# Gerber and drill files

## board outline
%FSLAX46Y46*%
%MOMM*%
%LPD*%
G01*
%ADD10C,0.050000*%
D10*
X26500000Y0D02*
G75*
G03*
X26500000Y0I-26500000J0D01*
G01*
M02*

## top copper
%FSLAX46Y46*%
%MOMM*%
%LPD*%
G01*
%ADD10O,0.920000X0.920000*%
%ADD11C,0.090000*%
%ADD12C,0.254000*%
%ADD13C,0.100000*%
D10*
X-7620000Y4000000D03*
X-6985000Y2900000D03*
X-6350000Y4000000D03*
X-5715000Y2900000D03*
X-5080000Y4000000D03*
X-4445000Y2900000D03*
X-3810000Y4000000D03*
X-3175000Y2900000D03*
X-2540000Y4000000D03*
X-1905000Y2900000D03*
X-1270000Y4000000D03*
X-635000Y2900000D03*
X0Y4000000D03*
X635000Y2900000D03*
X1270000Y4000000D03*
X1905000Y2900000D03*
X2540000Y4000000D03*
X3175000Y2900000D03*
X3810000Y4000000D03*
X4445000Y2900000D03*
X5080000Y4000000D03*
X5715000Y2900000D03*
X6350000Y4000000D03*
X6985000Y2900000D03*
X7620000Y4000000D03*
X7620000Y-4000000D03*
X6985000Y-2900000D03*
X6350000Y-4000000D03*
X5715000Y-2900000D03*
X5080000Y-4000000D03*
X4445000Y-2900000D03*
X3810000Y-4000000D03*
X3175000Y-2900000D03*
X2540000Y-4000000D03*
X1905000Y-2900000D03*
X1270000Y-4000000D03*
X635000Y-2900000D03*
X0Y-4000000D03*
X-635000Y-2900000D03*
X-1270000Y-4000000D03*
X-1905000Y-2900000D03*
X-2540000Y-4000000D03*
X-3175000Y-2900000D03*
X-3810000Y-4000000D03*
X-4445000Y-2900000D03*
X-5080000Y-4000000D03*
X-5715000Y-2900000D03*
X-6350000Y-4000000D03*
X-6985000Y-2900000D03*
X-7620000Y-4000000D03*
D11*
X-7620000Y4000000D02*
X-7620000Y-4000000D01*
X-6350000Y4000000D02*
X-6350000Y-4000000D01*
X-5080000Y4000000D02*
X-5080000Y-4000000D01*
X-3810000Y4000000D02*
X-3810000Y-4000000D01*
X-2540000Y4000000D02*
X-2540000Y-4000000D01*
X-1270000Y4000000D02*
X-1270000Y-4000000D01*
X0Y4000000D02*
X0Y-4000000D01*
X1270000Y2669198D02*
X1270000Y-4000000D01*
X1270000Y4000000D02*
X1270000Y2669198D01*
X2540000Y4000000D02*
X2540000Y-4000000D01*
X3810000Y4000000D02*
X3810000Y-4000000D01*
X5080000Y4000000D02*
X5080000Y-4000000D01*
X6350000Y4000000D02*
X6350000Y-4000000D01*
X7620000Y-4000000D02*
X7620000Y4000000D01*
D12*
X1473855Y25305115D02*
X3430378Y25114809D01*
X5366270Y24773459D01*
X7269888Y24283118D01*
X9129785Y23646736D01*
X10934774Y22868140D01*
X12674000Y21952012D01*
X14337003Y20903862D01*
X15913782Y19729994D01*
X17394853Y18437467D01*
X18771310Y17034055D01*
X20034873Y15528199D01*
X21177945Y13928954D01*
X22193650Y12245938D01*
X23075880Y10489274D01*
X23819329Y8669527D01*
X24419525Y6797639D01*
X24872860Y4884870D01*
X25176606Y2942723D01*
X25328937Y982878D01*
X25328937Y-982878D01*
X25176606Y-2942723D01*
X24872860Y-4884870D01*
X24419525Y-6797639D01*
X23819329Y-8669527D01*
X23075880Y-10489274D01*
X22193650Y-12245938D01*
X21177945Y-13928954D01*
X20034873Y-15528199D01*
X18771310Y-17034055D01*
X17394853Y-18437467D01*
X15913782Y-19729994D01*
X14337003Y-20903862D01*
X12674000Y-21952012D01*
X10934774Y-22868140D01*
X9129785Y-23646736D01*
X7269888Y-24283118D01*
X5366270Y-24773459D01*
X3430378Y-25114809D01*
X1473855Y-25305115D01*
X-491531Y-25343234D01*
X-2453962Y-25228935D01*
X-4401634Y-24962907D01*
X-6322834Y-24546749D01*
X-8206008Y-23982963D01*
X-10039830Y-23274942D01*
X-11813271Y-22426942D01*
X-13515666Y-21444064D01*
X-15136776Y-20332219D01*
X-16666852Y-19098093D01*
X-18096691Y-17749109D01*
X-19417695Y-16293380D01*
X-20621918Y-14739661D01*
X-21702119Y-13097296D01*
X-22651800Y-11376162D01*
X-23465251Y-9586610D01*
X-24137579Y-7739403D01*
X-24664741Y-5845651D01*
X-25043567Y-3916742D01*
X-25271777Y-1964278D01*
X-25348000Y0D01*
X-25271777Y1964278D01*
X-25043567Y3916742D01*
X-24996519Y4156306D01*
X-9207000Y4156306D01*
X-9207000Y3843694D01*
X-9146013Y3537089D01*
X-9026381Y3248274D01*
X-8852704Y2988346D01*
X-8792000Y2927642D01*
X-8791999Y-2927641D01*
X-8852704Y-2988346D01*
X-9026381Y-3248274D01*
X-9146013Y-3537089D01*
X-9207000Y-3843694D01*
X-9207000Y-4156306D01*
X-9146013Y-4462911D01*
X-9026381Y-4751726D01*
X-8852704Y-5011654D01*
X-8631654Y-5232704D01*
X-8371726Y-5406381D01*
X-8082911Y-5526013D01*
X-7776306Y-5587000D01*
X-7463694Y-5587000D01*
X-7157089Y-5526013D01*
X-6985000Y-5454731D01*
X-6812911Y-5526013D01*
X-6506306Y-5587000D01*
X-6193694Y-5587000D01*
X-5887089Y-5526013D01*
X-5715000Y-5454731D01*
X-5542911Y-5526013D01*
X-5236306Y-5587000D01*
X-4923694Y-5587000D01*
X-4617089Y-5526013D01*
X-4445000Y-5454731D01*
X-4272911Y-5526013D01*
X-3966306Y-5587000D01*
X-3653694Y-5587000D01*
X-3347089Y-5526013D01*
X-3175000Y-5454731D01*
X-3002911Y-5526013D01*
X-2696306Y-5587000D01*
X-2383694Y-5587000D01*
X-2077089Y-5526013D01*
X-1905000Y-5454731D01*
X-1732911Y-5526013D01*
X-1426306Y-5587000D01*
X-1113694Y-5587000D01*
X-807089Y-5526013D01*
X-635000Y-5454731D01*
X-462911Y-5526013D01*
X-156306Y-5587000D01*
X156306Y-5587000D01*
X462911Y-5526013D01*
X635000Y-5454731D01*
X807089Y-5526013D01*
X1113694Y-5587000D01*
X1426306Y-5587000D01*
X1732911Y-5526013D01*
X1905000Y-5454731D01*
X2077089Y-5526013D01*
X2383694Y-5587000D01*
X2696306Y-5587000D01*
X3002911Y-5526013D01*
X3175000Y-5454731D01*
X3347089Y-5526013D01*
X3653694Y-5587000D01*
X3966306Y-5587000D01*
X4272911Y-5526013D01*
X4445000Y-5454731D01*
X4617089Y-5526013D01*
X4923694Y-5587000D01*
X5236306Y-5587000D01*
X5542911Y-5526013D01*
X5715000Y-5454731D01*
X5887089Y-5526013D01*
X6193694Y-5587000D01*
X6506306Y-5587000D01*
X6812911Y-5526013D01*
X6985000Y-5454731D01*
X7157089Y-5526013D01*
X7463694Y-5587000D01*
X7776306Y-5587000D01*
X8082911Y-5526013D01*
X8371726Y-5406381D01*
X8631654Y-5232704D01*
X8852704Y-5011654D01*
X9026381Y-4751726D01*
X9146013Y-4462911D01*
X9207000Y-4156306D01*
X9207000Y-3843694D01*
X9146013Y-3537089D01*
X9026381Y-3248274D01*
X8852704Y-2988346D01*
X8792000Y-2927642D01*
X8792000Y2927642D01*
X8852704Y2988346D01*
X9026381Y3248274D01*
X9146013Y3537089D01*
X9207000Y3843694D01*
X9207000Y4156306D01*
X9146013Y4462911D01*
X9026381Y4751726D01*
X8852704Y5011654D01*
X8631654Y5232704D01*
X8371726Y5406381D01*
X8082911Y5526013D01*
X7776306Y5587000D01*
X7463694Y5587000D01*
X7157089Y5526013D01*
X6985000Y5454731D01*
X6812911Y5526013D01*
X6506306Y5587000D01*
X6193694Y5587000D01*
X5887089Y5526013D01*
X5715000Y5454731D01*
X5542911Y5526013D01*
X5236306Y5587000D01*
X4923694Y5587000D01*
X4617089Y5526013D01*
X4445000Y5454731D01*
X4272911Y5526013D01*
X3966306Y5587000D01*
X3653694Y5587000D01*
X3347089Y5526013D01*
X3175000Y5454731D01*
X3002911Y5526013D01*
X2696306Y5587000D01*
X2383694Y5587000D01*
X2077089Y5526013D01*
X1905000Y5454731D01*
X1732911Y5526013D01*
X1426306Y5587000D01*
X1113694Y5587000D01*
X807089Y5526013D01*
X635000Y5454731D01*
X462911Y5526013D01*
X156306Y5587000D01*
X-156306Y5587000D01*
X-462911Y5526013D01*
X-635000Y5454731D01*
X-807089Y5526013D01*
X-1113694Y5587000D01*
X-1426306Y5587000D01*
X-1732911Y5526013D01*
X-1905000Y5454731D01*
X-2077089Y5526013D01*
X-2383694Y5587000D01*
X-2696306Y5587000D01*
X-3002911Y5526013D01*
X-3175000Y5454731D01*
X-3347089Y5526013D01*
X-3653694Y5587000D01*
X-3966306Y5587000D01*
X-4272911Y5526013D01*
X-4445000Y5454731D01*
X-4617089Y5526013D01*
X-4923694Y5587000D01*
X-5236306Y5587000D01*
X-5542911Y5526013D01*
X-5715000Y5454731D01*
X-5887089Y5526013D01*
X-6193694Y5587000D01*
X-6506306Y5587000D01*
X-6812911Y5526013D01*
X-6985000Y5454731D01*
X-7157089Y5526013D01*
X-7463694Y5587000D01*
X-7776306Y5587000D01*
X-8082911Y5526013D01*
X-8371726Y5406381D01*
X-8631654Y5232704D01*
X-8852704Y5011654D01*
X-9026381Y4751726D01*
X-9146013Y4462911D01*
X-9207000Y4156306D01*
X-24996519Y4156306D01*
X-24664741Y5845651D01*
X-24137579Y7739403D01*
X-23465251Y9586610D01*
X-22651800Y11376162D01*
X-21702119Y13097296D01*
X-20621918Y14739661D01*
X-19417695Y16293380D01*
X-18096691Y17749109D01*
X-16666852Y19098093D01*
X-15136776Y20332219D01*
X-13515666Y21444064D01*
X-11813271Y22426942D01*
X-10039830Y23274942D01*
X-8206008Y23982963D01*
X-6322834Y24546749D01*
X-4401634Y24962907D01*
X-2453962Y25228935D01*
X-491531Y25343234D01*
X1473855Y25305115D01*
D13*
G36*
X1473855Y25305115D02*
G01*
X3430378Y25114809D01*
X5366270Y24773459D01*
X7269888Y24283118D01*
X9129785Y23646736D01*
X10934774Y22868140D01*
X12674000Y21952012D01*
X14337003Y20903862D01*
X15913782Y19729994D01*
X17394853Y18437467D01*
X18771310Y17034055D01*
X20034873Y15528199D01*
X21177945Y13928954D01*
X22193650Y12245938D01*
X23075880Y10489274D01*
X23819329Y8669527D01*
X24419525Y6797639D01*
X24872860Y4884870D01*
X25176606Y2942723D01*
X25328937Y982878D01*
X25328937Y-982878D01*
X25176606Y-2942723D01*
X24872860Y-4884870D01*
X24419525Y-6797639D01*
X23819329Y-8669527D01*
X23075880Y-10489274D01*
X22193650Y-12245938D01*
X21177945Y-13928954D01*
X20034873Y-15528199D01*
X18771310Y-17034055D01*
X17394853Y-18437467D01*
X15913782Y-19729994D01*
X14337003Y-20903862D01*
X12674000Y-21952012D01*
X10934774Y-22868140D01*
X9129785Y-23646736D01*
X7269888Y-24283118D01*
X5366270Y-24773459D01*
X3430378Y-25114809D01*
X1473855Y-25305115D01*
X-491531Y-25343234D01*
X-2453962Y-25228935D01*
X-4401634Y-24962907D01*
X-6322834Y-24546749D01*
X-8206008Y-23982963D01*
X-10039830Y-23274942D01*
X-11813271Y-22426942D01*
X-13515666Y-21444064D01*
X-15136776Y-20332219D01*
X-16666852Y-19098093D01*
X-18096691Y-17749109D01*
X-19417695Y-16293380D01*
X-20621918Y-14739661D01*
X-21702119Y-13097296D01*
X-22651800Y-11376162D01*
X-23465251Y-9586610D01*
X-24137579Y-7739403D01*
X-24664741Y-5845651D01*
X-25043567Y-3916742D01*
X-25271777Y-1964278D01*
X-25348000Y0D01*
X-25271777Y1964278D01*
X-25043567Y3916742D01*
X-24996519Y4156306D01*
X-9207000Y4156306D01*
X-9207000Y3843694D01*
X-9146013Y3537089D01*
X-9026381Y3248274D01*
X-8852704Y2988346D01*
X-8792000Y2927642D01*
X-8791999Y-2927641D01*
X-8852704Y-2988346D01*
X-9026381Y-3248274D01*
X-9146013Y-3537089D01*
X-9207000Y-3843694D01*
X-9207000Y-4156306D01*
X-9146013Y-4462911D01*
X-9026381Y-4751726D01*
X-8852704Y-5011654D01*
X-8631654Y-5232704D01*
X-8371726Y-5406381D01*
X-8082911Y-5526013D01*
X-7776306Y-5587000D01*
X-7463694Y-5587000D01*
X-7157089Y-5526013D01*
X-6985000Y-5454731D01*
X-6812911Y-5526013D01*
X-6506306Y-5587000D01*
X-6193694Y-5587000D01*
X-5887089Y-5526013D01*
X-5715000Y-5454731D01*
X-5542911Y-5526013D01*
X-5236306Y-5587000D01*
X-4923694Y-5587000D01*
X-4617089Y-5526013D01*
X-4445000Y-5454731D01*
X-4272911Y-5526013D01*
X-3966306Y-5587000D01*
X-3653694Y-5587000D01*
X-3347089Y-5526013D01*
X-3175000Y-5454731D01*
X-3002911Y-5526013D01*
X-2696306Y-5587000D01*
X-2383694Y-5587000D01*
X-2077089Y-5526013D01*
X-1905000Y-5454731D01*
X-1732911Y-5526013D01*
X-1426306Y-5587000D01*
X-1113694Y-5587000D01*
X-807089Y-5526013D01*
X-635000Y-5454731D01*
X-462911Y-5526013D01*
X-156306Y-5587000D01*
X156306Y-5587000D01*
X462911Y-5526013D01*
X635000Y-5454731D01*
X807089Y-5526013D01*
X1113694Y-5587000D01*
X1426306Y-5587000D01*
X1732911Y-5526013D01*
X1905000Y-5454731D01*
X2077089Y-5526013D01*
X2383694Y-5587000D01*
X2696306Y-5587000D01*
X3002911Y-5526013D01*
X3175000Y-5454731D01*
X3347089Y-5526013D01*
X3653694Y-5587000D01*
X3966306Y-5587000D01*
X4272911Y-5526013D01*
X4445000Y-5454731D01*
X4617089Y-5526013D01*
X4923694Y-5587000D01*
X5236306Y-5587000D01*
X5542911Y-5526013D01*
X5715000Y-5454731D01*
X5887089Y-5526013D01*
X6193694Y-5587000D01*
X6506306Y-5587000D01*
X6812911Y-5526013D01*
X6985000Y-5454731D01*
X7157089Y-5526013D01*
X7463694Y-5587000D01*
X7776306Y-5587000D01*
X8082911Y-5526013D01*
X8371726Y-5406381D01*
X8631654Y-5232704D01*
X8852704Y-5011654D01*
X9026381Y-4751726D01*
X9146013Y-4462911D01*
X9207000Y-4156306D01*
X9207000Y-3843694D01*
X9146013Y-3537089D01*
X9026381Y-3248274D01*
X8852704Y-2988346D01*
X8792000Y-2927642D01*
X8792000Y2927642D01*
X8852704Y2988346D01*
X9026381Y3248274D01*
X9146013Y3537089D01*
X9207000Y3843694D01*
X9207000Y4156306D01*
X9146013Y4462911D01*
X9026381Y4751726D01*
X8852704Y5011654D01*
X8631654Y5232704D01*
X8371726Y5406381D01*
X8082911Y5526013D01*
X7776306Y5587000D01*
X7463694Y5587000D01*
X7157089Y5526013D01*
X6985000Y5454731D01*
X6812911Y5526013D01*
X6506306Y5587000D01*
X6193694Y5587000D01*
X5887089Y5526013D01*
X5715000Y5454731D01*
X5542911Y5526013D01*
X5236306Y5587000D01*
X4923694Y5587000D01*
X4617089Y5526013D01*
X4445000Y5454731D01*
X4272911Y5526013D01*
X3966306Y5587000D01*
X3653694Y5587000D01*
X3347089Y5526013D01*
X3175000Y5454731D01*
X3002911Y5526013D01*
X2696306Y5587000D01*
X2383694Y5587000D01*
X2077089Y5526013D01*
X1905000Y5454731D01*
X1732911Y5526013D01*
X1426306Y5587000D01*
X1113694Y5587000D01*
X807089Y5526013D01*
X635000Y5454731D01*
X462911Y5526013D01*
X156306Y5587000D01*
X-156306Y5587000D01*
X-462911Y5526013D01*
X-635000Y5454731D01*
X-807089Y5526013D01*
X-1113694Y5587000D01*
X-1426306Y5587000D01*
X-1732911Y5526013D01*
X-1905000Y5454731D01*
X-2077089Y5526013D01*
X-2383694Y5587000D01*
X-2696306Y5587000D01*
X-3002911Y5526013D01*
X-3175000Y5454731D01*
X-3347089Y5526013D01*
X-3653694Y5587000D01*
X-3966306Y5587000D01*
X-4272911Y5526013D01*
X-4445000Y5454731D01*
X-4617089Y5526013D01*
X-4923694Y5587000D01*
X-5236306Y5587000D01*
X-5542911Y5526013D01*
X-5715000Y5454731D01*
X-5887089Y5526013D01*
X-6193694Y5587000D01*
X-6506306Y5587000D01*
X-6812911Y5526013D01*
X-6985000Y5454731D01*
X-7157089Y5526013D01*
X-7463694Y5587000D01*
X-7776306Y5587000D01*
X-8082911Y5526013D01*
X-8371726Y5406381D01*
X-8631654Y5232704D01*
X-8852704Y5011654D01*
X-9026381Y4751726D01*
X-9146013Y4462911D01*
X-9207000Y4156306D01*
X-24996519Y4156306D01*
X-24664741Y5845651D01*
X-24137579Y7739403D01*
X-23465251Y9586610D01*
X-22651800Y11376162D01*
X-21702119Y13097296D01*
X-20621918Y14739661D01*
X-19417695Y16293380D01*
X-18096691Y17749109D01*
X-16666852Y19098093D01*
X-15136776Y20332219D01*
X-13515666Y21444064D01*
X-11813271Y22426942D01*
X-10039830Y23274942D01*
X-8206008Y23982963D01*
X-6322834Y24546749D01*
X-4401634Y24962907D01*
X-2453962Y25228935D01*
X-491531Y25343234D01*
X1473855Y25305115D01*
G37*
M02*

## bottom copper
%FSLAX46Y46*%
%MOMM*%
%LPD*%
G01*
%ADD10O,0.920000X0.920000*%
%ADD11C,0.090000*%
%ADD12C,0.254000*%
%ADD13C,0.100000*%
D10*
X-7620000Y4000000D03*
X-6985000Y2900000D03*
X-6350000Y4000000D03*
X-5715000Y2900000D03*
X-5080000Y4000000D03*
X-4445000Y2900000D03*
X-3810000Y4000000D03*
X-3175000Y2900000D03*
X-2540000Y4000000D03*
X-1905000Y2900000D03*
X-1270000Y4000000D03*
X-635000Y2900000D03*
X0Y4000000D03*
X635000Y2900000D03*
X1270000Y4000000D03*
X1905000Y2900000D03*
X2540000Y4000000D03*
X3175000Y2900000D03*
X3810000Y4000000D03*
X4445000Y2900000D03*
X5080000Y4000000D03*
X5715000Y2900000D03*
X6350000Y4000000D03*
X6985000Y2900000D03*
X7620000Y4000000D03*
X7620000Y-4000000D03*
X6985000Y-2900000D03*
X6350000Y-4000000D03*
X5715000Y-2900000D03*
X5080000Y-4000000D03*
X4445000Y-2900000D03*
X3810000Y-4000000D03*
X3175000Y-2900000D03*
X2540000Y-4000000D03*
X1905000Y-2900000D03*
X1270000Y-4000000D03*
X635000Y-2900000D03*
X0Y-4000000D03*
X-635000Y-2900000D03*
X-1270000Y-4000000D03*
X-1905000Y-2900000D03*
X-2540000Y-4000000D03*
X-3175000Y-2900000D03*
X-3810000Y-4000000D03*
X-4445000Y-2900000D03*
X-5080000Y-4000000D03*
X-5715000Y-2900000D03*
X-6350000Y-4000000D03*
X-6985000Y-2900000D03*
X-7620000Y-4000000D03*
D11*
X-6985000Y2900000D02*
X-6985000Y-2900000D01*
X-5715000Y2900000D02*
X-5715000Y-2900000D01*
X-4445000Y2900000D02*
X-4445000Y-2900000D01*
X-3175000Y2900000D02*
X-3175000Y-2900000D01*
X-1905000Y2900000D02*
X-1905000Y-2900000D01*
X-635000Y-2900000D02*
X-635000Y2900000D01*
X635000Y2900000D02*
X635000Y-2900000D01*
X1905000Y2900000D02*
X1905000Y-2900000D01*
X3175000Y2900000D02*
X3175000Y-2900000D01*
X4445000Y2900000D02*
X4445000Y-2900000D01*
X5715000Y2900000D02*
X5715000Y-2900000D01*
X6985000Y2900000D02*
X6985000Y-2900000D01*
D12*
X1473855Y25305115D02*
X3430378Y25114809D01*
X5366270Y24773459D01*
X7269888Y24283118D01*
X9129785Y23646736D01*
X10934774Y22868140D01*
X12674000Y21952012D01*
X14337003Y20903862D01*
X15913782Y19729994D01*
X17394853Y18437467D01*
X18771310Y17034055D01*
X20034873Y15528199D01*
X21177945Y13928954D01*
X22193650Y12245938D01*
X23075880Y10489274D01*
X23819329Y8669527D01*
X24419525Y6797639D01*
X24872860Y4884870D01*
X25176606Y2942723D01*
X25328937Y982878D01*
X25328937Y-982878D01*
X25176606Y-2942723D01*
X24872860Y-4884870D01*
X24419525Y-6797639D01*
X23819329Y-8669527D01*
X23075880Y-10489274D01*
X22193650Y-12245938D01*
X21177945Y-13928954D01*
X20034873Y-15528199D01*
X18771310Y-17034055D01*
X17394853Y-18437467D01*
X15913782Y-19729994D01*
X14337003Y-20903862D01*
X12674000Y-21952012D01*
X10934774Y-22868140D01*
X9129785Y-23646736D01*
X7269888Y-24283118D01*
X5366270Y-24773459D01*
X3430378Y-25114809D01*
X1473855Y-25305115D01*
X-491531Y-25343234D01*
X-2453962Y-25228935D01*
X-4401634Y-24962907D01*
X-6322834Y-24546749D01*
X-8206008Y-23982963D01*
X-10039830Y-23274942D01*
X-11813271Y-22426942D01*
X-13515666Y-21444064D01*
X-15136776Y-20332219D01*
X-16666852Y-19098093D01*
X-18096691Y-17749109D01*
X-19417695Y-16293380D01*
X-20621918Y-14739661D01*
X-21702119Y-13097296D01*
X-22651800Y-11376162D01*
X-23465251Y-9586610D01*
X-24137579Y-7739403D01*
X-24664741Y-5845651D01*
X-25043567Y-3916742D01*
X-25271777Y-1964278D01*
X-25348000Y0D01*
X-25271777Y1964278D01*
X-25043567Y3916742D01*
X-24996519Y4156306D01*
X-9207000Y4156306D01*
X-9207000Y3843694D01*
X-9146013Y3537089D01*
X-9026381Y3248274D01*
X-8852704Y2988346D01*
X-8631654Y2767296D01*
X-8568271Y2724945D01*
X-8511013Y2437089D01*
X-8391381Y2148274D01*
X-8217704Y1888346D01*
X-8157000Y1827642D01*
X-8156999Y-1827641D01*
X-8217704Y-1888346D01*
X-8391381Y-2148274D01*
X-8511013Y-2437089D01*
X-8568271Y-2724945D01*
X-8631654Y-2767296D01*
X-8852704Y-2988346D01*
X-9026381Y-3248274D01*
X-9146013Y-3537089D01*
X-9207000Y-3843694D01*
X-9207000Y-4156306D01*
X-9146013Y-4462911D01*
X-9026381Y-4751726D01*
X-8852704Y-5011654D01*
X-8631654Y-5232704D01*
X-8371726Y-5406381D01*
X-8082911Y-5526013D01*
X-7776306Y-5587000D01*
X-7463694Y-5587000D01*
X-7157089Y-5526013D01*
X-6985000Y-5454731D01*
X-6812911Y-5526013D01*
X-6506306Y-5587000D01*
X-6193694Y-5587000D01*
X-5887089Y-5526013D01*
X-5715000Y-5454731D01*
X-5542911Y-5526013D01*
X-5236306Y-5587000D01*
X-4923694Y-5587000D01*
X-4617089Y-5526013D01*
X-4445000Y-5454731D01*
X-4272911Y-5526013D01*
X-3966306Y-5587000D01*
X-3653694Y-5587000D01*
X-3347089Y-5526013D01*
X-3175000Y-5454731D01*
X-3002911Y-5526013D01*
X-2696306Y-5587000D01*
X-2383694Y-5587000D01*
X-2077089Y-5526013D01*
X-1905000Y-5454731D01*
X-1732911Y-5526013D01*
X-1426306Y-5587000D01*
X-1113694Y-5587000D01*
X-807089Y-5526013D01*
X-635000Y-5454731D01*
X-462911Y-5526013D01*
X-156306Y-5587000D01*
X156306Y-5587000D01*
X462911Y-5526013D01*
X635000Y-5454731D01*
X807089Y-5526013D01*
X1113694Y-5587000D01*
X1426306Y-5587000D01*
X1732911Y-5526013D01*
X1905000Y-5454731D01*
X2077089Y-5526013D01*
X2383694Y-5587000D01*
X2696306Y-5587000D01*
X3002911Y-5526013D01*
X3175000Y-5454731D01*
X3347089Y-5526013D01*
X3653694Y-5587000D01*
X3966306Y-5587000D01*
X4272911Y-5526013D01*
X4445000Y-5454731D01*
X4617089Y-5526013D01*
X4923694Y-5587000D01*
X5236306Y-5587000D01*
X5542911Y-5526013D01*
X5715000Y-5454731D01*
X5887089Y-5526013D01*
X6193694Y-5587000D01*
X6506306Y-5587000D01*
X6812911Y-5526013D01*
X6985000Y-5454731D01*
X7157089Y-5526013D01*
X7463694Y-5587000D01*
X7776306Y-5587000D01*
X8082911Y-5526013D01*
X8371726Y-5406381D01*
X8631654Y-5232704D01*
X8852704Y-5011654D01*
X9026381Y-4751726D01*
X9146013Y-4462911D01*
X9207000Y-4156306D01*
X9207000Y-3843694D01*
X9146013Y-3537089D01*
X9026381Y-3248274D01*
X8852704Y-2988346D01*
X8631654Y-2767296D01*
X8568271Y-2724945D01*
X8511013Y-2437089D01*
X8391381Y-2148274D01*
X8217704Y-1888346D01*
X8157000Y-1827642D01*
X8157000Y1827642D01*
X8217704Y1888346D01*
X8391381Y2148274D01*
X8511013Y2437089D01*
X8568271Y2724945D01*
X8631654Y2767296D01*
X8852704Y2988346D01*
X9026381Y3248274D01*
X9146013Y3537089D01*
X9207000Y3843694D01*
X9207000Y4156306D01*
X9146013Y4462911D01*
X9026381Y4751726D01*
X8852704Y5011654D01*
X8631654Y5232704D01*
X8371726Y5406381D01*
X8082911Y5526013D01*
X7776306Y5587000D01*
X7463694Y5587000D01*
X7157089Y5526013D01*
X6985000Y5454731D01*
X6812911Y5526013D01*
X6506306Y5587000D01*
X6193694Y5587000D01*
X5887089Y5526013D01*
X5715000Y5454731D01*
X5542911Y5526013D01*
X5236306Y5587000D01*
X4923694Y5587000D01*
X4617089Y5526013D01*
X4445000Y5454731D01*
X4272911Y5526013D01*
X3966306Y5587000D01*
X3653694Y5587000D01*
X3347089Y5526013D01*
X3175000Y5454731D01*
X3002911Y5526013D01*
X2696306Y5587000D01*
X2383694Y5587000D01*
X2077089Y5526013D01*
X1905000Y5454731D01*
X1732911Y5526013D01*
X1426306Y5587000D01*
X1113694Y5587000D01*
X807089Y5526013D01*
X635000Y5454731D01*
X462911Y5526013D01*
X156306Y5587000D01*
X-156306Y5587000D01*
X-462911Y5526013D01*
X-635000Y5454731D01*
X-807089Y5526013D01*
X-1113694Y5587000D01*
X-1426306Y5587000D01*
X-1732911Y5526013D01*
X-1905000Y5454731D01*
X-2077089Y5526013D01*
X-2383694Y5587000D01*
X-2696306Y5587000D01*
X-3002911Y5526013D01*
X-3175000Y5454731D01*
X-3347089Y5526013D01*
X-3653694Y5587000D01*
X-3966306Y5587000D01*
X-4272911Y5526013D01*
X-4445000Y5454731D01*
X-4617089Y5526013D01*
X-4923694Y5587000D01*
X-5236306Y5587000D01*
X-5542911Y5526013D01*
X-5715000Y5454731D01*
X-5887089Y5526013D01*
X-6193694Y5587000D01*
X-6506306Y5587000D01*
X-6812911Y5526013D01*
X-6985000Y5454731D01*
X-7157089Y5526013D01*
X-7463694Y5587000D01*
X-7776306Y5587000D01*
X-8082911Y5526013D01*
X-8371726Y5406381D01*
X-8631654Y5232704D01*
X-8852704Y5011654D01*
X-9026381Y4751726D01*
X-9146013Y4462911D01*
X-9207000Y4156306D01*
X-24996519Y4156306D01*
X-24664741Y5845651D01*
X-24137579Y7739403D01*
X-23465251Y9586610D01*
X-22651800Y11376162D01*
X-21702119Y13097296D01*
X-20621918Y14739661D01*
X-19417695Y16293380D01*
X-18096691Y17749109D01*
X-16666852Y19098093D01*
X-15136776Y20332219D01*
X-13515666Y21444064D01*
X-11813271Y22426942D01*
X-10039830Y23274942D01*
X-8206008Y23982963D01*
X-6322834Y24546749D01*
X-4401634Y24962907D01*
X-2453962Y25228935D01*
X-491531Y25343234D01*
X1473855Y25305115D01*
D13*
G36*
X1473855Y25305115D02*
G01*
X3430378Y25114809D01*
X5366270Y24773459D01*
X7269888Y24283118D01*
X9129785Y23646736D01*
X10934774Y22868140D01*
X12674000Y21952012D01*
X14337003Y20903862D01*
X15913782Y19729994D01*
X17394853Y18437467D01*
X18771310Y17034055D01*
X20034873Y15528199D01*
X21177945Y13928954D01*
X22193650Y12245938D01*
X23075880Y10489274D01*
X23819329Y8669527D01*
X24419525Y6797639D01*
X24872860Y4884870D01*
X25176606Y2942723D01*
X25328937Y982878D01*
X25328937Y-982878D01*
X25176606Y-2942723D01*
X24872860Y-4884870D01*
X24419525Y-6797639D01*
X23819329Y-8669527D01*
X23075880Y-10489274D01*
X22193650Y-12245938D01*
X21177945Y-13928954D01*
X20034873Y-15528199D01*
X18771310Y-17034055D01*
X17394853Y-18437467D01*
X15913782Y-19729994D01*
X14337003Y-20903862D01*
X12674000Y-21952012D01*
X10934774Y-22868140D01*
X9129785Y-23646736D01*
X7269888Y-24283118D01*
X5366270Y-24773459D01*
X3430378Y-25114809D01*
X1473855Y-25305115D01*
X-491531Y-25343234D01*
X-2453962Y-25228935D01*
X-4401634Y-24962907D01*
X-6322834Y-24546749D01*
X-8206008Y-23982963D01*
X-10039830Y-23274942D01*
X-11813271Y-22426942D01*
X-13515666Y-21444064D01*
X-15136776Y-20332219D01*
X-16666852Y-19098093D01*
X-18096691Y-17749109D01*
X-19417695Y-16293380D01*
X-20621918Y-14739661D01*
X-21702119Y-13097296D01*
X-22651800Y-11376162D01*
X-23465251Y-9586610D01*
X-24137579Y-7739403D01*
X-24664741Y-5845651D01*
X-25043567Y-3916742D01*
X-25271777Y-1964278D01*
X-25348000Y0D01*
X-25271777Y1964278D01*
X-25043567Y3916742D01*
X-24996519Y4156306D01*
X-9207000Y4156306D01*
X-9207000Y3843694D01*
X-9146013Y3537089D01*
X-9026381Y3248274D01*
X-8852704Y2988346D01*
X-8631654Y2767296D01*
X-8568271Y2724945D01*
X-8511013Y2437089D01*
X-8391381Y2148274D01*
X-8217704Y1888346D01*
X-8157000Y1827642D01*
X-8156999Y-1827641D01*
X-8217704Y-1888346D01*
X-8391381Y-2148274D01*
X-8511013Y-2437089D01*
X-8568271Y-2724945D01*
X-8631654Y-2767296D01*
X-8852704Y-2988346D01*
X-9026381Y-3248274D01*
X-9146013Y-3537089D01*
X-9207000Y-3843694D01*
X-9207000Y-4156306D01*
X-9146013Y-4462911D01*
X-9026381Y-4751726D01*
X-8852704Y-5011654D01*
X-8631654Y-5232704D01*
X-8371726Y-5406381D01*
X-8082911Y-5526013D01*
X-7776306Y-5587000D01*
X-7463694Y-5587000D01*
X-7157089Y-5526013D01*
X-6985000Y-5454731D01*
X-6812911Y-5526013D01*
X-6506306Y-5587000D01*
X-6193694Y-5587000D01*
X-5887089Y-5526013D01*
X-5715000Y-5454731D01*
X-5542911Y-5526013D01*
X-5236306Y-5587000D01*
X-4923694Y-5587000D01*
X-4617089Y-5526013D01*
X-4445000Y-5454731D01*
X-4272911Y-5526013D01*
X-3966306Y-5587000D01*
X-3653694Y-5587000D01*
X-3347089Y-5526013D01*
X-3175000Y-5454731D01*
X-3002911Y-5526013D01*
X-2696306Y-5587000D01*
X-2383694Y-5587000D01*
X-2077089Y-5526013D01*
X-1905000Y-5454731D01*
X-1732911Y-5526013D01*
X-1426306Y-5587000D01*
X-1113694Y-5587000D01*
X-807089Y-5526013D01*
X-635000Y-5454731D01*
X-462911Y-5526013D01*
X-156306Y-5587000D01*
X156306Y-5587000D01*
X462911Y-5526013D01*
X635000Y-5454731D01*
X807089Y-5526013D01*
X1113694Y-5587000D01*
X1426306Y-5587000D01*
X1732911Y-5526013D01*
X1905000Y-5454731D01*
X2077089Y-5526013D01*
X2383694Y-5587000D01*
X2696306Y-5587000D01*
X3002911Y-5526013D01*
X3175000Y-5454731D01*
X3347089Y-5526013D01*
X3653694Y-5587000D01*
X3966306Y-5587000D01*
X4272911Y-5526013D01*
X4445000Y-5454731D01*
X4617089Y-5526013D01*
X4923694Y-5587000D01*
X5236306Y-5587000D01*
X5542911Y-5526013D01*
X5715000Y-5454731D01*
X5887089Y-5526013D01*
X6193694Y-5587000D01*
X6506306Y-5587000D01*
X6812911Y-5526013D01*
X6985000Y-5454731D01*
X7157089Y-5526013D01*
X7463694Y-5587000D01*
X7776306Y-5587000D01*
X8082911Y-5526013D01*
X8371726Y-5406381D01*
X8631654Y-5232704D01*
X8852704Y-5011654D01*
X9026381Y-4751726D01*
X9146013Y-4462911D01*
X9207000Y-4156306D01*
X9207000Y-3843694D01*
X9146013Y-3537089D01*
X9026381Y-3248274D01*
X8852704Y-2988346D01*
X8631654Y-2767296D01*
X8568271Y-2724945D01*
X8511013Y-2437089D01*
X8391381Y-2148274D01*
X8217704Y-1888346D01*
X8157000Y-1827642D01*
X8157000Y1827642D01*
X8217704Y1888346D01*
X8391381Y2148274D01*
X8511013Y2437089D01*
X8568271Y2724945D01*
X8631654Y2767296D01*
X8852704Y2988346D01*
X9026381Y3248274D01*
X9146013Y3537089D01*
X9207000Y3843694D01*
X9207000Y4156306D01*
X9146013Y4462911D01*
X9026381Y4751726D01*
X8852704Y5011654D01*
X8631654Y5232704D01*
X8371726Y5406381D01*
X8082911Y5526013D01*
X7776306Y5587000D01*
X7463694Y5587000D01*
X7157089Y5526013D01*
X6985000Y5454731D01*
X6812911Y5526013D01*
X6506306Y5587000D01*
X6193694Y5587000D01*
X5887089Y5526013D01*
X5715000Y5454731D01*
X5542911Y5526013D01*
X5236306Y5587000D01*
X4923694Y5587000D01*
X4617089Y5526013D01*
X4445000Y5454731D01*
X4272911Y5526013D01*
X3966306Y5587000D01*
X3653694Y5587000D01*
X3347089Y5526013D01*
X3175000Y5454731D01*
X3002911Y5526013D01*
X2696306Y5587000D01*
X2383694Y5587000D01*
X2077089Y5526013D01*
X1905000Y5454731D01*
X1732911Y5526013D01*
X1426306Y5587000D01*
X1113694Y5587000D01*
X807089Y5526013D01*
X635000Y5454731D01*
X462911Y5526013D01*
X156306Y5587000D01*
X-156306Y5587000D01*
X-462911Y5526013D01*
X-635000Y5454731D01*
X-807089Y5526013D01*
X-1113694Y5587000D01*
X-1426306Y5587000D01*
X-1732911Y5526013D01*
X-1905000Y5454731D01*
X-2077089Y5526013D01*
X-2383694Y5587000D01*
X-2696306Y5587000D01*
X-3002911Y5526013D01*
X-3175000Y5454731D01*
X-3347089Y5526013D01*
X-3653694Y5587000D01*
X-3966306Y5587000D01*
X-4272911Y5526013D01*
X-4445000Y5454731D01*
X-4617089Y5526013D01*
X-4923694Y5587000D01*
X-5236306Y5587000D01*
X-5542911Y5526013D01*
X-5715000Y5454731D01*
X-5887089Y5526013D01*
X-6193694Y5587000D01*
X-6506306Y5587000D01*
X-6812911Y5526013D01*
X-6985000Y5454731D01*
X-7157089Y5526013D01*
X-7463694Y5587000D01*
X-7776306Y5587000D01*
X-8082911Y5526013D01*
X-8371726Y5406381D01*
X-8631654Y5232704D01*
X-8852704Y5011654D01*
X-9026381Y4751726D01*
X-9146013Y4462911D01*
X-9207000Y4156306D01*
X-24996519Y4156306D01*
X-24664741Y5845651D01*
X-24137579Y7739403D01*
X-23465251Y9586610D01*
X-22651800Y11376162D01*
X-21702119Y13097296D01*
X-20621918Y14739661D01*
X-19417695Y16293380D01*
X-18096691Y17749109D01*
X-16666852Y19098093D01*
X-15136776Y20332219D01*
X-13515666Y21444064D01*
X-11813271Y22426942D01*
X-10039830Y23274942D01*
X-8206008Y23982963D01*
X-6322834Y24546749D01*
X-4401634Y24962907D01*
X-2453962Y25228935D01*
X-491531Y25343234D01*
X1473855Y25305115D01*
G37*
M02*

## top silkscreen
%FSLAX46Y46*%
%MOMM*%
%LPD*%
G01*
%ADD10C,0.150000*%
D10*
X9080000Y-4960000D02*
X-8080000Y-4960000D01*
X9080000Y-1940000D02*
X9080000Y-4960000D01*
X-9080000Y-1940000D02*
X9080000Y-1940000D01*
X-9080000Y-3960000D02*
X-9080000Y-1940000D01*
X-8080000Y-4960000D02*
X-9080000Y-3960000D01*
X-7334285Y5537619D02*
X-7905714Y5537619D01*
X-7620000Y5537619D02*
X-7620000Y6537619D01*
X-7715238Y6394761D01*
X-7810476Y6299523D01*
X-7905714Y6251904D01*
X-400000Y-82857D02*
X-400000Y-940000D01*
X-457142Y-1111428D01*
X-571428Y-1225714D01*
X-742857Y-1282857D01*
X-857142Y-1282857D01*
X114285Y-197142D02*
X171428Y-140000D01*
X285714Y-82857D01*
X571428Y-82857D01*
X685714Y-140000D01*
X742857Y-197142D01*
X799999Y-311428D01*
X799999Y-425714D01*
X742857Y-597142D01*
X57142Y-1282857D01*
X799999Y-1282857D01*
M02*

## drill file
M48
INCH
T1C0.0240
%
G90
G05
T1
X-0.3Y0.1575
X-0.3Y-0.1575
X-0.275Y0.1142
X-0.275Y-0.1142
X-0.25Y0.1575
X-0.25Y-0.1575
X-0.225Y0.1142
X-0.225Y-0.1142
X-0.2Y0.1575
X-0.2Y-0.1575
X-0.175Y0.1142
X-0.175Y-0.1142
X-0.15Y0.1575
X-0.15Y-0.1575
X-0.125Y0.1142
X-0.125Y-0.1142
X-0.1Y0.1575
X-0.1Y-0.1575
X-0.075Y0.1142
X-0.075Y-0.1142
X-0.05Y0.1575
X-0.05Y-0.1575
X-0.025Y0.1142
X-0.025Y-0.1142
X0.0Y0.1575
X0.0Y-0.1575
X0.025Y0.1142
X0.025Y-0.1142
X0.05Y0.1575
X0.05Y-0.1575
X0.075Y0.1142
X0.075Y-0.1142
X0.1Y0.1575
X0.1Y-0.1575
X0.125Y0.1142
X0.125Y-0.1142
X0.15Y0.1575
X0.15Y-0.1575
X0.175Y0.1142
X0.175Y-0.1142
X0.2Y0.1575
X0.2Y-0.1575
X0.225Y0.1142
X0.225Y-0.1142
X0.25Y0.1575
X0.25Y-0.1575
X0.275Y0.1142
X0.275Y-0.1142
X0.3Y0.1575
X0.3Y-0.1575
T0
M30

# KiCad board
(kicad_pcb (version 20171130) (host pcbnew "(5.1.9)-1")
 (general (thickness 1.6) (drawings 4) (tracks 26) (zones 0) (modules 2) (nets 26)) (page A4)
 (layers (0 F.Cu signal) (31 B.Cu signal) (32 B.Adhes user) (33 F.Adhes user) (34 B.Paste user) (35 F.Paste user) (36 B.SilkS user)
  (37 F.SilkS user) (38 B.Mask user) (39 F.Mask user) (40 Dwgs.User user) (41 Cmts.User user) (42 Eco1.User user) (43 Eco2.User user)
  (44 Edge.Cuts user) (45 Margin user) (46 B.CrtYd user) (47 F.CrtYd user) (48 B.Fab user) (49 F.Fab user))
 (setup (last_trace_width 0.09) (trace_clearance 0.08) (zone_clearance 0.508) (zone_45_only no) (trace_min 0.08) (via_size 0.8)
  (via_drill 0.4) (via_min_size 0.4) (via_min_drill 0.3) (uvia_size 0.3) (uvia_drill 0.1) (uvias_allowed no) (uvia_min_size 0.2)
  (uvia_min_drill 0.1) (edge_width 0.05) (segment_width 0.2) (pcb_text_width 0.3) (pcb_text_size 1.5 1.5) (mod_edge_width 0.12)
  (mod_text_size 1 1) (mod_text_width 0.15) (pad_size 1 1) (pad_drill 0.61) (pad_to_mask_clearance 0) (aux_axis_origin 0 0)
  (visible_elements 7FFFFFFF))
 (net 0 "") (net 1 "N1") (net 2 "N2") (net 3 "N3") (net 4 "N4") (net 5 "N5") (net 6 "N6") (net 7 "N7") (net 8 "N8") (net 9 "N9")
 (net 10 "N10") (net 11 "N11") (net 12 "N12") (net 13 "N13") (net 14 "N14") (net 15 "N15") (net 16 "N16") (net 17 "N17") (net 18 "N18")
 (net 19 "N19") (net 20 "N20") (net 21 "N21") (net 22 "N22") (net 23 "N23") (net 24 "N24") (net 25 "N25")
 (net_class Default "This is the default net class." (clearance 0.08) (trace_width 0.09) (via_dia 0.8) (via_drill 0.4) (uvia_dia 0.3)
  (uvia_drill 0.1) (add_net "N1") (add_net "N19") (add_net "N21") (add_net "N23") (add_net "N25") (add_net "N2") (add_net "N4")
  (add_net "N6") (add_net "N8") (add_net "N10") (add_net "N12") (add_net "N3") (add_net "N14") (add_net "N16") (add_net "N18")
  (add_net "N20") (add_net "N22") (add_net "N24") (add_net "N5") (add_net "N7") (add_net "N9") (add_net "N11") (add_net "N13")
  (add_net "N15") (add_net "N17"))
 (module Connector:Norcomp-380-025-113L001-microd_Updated (layer F.Cu) (at 0 -3.45)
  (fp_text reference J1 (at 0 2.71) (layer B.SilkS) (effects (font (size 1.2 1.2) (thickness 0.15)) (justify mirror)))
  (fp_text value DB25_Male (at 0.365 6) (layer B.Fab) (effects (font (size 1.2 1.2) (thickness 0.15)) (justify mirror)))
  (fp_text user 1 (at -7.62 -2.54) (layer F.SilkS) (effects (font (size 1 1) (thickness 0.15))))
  (pad 1 thru_hole oval (at -7.62 -0.55) (size 0.92 0.92) (drill 0.61) (layers *.Cu *.Mask) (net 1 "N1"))
  (pad 14 thru_hole oval (at -6.985 0.55) (size 0.92 0.92) (drill 0.61) (layers *.Cu *.Mask) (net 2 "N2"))
  (pad 2 thru_hole oval (at -6.35 -0.55) (size 0.92 0.92) (drill 0.61) (layers *.Cu *.Mask) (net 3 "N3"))
  (pad 15 thru_hole oval (at -5.715 0.55) (size 0.92 0.92) (drill 0.61) (layers *.Cu *.Mask) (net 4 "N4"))
  (pad 3 thru_hole oval (at -5.08 -0.55) (size 0.92 0.92) (drill 0.61) (layers *.Cu *.Mask) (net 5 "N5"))
  (pad 16 thru_hole oval (at -4.445 0.55) (size 0.92 0.92) (drill 0.61) (layers *.Cu *.Mask) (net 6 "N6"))
  (pad 4 thru_hole oval (at -3.81 -0.55) (size 0.92 0.92) (drill 0.61) (layers *.Cu *.Mask) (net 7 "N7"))
  (pad 17 thru_hole oval (at -3.175 0.55) (size 0.92 0.92) (drill 0.61) (layers *.Cu *.Mask) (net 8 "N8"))
  (pad 5 thru_hole oval (at -2.54 -0.55) (size 0.92 0.92) (drill 0.61) (layers *.Cu *.Mask) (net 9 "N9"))
  (pad 18 thru_hole oval (at -1.905 0.55) (size 0.92 0.92) (drill 0.61) (layers *.Cu *.Mask) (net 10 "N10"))
  (pad 6 thru_hole oval (at -1.27 -0.55) (size 0.92 0.92) (drill 0.61) (layers *.Cu *.Mask) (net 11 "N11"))
  (pad 19 thru_hole oval (at -0.635 0.55) (size 0.92 0.92) (drill 0.61) (layers *.Cu *.Mask) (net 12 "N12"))
  (pad 7 thru_hole oval (at 0 -0.55) (size 0.92 0.92) (drill 0.61) (layers *.Cu *.Mask) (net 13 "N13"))
  (pad 20 thru_hole oval (at 0.635 0.55) (size 0.92 0.92) (drill 0.61) (layers *.Cu *.Mask) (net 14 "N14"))
  (pad 8 thru_hole oval (at 1.27 -0.55) (size 0.92 0.92) (drill 0.61) (layers *.Cu *.Mask) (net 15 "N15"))
  (pad 21 thru_hole oval (at 1.905 0.55) (size 0.92 0.92) (drill 0.61) (layers *.Cu *.Mask) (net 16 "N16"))
  (pad 9 thru_hole oval (at 2.54 -0.55) (size 0.92 0.92) (drill 0.61) (layers *.Cu *.Mask) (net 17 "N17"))
  (pad 22 thru_hole oval (at 3.175 0.55) (size 0.92 0.92) (drill 0.61) (layers *.Cu *.Mask) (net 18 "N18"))
  (pad 10 thru_hole oval (at 3.81 -0.55) (size 0.92 0.92) (drill 0.61) (layers *.Cu *.Mask) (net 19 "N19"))
  (pad 23 thru_hole oval (at 4.445 0.55) (size 0.92 0.92) (drill 0.61) (layers *.Cu *.Mask) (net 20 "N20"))
  (pad 11 thru_hole oval (at 5.08 -0.55) (size 0.92 0.92) (drill 0.61) (layers *.Cu *.Mask) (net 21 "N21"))
  (pad 24 thru_hole oval (at 5.715 0.55) (size 0.92 0.92) (drill 0.61) (layers *.Cu *.Mask) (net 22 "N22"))
  (pad 12 thru_hole oval (at 6.35 -0.55) (size 0.92 0.92) (drill 0.61) (layers *.Cu *.Mask) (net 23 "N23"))
  (pad 25 thru_hole oval (at 6.985 0.55) (size 0.92 0.92) (drill 0.61) (layers *.Cu *.Mask) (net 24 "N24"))
  (pad 13 thru_hole oval (at 7.62 -0.55) (size 0.92 0.92) (drill 0.61) (layers *.Cu *.Mask) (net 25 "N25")))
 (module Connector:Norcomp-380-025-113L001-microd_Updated (layer B.Cu) (at 0 3.45)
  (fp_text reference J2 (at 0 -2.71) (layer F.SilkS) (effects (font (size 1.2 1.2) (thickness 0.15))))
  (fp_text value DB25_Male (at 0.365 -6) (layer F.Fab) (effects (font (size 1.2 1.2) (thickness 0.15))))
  (fp_line (start 9.08 1.51) (end -8.08 1.51) (layer F.SilkS) (width 0.15))
  (fp_line (start 9.08 -1.51) (end 9.08 1.51) (layer F.SilkS) (width 0.15))
  (fp_line (start -9.08 -1.51) (end 9.08 -1.51) (layer F.SilkS) (width 0.15))
  (fp_line (start -9.08 0.51) (end -9.08 -1.51) (layer F.SilkS) (width 0.15))
  (fp_line (start -8.08 1.51) (end -9.08 0.51) (layer F.SilkS) (width 0.15))
  (pad 13 thru_hole oval (at 7.62 0.55) (size 0.92 0.92) (drill 0.61) (layers *.Cu *.Mask) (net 25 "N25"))
  (pad 25 thru_hole oval (at 6.985 -0.55) (size 0.92 0.92) (drill 0.61) (layers *.Cu *.Mask) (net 24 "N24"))
  (pad 12 thru_hole oval (at 6.35 0.55) (size 0.92 0.92) (drill 0.61) (layers *.Cu *.Mask) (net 23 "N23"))
  (pad 24 thru_hole oval (at 5.715 -0.55) (size 0.92 0.92) (drill 0.61) (layers *.Cu *.Mask) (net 22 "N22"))
  (pad 11 thru_hole oval (at 5.08 0.55) (size 0.92 0.92) (drill 0.61) (layers *.Cu *.Mask) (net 21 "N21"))
  (pad 23 thru_hole oval (at 4.445 -0.55) (size 0.92 0.92) (drill 0.61) (layers *.Cu *.Mask) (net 20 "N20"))
  (pad 10 thru_hole oval (at 3.81 0.55) (size 0.92 0.92) (drill 0.61) (layers *.Cu *.Mask) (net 19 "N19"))
  (pad 22 thru_hole oval (at 3.175 -0.55) (size 0.92 0.92) (drill 0.61) (layers *.Cu *.Mask) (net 18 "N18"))
  (pad 9 thru_hole oval (at 2.54 0.55) (size 0.92 0.92) (drill 0.61) (layers *.Cu *.Mask) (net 17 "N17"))
  (pad 21 thru_hole oval (at 1.905 -0.55) (size 0.92 0.92) (drill 0.61) (layers *.Cu *.Mask) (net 16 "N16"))
  (pad 8 thru_hole oval (at 1.27 0.55) (size 0.92 0.92) (drill 0.61) (layers *.Cu *.Mask) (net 15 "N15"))
  (pad 20 thru_hole oval (at 0.635 -0.55) (size 0.92 0.92) (drill 0.61) (layers *.Cu *.Mask) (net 14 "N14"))
  (pad 7 thru_hole oval (at 0 0.55) (size 0.92 0.92) (drill 0.61) (layers *.Cu *.Mask) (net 13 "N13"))
  (pad 19 thru_hole oval (at -0.635 -0.55) (size 0.92 0.92) (drill 0.61) (layers *.Cu *.Mask) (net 12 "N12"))
  (pad 6 thru_hole oval (at -1.27 0.55) (size 0.92 0.92) (drill 0.61) (layers *.Cu *.Mask) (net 11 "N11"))
  (pad 18 thru_hole oval (at -1.905 -0.55) (size 0.92 0.92) (drill 0.61) (layers *.Cu *.Mask) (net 10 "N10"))
  (pad 5 thru_hole oval (at -2.54 0.55) (size 0.92 0.92) (drill 0.61) (layers *.Cu *.Mask) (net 9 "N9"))
  (pad 17 thru_hole oval (at -3.175 -0.55) (size 0.92 0.92) (drill 0.61) (layers *.Cu *.Mask) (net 8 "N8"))
  (pad 4 thru_hole oval (at -3.81 0.55) (size 0.92 0.92) (drill 0.61) (layers *.Cu *.Mask) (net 7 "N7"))
  (pad 16 thru_hole oval (at -4.445 -0.55) (size 0.92 0.92) (drill 0.61) (layers *.Cu *.Mask) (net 6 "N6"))
  (pad 3 thru_hole oval (at -5.08 0.55) (size 0.92 0.92) (drill 0.61) (layers *.Cu *.Mask) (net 5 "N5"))
  (pad 15 thru_hole oval (at -5.715 -0.55) (size 0.92 0.92) (drill 0.61) (layers *.Cu *.Mask) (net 4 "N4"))
  (pad 2 thru_hole oval (at -6.35 0.55) (size 0.92 0.92) (drill 0.61) (layers *.Cu *.Mask) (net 3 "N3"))
  (pad 14 thru_hole oval (at -6.985 -0.55) (size 0.92 0.92) (drill 0.61) (layers *.Cu *.Mask) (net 2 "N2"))
  (pad 1 thru_hole oval (at -7.62 0.55) (size 0.92 0.92) (drill 0.61) (layers *.Cu *.Mask) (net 1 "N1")))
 (gr_circle (center 0 0) (end 26.5 0) (layer Edge.Cuts) (width 0.05))
 (segment (start -7.62 -4) (end -7.62 4) (width 0.09) (layer F.Cu) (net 1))
 (segment (start -6.985 -2.9) (end -6.985 2.9) (width 0.09) (layer B.Cu) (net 2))
 (segment (start -6.35 -4) (end -6.35 4) (width 0.09) (layer F.Cu) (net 3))
 (segment (start -5.08 -4) (end -5.08 4) (width 0.09) (layer F.Cu) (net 5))
 (segment (start -3.81 -4) (end -3.81 4) (width 0.09) (layer F.Cu) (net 7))
 (segment (start -2.54 -4) (end -2.54 4) (width 0.09) (layer F.Cu) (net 9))
 (segment (start -1.27 -4) (end -1.27 4) (width 0.09) (layer F.Cu) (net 11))
 (segment (start 0 -4) (end 0 4) (width 0.09) (layer F.Cu) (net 13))
 (segment (start 1.27 -2.669198) (end 1.27 4) (width 0.09) (layer F.Cu) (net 15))
 (segment (start 1.27 -4) (end 1.27 -2.669198) (width 0.09) (layer F.Cu) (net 15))
 (segment (start 2.54 -4) (end 2.54 4) (width 0.09) (layer F.Cu) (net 17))
 (segment (start 3.81 -4) (end 3.81 4) (width 0.09) (layer F.Cu) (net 19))
 (segment (start 5.08 -4) (end 5.08 4) (width 0.09) (layer F.Cu) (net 21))
 (segment (start 6.35 -4) (end 6.35 4) (width 0.09) (layer F.Cu) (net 23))
 (segment (start 7.62 4) (end 7.62 -4) (width 0.09) (layer F.Cu) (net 25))
 (segment (start -5.715 -2.9) (end -5.715 2.9) (width 0.09) (layer B.Cu) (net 4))
 (segment (start -4.445 -2.9) (end -4.445 2.9) (width 0.09) (layer B.Cu) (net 6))
 (segment (start -3.175 -2.9) (end -3.175 2.9) (width 0.09) (layer B.Cu) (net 8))
 (segment (start -1.905 -2.9) (end -1.905 2.9) (width 0.09) (layer B.Cu) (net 10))
 (segment (start -0.635 2.9) (end -0.635 -2.9) (width 0.09) (layer B.Cu) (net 12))
 (segment (start 0.635 -2.9) (end 0.635 2.9) (width 0.09) (layer B.Cu) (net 14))
 (segment (start 1.905 -2.9) (end 1.905 2.9) (width 0.09) (layer B.Cu) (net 16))
 (segment (start 3.175 -2.9) (end 3.175 2.9) (width 0.09) (layer B.Cu) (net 18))
 (segment (start 4.445 -2.9) (end 4.445 2.9) (width 0.09) (layer B.Cu) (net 20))
 (segment (start 5.715 -2.9) (end 5.715 2.9) (width 0.09) (layer B.Cu) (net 22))
 (segment (start 6.985 -2.9) (end 6.985 2.9) (width 0.09) (layer B.Cu) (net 24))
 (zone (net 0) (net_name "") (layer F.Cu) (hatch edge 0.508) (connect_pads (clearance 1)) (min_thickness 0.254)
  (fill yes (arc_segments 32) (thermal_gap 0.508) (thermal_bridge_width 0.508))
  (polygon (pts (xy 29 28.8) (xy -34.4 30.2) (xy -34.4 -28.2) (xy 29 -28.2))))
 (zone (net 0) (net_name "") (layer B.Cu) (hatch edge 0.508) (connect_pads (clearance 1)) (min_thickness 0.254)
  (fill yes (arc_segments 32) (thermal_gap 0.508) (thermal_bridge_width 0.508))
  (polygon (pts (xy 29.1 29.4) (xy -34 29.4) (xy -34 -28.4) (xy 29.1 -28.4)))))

